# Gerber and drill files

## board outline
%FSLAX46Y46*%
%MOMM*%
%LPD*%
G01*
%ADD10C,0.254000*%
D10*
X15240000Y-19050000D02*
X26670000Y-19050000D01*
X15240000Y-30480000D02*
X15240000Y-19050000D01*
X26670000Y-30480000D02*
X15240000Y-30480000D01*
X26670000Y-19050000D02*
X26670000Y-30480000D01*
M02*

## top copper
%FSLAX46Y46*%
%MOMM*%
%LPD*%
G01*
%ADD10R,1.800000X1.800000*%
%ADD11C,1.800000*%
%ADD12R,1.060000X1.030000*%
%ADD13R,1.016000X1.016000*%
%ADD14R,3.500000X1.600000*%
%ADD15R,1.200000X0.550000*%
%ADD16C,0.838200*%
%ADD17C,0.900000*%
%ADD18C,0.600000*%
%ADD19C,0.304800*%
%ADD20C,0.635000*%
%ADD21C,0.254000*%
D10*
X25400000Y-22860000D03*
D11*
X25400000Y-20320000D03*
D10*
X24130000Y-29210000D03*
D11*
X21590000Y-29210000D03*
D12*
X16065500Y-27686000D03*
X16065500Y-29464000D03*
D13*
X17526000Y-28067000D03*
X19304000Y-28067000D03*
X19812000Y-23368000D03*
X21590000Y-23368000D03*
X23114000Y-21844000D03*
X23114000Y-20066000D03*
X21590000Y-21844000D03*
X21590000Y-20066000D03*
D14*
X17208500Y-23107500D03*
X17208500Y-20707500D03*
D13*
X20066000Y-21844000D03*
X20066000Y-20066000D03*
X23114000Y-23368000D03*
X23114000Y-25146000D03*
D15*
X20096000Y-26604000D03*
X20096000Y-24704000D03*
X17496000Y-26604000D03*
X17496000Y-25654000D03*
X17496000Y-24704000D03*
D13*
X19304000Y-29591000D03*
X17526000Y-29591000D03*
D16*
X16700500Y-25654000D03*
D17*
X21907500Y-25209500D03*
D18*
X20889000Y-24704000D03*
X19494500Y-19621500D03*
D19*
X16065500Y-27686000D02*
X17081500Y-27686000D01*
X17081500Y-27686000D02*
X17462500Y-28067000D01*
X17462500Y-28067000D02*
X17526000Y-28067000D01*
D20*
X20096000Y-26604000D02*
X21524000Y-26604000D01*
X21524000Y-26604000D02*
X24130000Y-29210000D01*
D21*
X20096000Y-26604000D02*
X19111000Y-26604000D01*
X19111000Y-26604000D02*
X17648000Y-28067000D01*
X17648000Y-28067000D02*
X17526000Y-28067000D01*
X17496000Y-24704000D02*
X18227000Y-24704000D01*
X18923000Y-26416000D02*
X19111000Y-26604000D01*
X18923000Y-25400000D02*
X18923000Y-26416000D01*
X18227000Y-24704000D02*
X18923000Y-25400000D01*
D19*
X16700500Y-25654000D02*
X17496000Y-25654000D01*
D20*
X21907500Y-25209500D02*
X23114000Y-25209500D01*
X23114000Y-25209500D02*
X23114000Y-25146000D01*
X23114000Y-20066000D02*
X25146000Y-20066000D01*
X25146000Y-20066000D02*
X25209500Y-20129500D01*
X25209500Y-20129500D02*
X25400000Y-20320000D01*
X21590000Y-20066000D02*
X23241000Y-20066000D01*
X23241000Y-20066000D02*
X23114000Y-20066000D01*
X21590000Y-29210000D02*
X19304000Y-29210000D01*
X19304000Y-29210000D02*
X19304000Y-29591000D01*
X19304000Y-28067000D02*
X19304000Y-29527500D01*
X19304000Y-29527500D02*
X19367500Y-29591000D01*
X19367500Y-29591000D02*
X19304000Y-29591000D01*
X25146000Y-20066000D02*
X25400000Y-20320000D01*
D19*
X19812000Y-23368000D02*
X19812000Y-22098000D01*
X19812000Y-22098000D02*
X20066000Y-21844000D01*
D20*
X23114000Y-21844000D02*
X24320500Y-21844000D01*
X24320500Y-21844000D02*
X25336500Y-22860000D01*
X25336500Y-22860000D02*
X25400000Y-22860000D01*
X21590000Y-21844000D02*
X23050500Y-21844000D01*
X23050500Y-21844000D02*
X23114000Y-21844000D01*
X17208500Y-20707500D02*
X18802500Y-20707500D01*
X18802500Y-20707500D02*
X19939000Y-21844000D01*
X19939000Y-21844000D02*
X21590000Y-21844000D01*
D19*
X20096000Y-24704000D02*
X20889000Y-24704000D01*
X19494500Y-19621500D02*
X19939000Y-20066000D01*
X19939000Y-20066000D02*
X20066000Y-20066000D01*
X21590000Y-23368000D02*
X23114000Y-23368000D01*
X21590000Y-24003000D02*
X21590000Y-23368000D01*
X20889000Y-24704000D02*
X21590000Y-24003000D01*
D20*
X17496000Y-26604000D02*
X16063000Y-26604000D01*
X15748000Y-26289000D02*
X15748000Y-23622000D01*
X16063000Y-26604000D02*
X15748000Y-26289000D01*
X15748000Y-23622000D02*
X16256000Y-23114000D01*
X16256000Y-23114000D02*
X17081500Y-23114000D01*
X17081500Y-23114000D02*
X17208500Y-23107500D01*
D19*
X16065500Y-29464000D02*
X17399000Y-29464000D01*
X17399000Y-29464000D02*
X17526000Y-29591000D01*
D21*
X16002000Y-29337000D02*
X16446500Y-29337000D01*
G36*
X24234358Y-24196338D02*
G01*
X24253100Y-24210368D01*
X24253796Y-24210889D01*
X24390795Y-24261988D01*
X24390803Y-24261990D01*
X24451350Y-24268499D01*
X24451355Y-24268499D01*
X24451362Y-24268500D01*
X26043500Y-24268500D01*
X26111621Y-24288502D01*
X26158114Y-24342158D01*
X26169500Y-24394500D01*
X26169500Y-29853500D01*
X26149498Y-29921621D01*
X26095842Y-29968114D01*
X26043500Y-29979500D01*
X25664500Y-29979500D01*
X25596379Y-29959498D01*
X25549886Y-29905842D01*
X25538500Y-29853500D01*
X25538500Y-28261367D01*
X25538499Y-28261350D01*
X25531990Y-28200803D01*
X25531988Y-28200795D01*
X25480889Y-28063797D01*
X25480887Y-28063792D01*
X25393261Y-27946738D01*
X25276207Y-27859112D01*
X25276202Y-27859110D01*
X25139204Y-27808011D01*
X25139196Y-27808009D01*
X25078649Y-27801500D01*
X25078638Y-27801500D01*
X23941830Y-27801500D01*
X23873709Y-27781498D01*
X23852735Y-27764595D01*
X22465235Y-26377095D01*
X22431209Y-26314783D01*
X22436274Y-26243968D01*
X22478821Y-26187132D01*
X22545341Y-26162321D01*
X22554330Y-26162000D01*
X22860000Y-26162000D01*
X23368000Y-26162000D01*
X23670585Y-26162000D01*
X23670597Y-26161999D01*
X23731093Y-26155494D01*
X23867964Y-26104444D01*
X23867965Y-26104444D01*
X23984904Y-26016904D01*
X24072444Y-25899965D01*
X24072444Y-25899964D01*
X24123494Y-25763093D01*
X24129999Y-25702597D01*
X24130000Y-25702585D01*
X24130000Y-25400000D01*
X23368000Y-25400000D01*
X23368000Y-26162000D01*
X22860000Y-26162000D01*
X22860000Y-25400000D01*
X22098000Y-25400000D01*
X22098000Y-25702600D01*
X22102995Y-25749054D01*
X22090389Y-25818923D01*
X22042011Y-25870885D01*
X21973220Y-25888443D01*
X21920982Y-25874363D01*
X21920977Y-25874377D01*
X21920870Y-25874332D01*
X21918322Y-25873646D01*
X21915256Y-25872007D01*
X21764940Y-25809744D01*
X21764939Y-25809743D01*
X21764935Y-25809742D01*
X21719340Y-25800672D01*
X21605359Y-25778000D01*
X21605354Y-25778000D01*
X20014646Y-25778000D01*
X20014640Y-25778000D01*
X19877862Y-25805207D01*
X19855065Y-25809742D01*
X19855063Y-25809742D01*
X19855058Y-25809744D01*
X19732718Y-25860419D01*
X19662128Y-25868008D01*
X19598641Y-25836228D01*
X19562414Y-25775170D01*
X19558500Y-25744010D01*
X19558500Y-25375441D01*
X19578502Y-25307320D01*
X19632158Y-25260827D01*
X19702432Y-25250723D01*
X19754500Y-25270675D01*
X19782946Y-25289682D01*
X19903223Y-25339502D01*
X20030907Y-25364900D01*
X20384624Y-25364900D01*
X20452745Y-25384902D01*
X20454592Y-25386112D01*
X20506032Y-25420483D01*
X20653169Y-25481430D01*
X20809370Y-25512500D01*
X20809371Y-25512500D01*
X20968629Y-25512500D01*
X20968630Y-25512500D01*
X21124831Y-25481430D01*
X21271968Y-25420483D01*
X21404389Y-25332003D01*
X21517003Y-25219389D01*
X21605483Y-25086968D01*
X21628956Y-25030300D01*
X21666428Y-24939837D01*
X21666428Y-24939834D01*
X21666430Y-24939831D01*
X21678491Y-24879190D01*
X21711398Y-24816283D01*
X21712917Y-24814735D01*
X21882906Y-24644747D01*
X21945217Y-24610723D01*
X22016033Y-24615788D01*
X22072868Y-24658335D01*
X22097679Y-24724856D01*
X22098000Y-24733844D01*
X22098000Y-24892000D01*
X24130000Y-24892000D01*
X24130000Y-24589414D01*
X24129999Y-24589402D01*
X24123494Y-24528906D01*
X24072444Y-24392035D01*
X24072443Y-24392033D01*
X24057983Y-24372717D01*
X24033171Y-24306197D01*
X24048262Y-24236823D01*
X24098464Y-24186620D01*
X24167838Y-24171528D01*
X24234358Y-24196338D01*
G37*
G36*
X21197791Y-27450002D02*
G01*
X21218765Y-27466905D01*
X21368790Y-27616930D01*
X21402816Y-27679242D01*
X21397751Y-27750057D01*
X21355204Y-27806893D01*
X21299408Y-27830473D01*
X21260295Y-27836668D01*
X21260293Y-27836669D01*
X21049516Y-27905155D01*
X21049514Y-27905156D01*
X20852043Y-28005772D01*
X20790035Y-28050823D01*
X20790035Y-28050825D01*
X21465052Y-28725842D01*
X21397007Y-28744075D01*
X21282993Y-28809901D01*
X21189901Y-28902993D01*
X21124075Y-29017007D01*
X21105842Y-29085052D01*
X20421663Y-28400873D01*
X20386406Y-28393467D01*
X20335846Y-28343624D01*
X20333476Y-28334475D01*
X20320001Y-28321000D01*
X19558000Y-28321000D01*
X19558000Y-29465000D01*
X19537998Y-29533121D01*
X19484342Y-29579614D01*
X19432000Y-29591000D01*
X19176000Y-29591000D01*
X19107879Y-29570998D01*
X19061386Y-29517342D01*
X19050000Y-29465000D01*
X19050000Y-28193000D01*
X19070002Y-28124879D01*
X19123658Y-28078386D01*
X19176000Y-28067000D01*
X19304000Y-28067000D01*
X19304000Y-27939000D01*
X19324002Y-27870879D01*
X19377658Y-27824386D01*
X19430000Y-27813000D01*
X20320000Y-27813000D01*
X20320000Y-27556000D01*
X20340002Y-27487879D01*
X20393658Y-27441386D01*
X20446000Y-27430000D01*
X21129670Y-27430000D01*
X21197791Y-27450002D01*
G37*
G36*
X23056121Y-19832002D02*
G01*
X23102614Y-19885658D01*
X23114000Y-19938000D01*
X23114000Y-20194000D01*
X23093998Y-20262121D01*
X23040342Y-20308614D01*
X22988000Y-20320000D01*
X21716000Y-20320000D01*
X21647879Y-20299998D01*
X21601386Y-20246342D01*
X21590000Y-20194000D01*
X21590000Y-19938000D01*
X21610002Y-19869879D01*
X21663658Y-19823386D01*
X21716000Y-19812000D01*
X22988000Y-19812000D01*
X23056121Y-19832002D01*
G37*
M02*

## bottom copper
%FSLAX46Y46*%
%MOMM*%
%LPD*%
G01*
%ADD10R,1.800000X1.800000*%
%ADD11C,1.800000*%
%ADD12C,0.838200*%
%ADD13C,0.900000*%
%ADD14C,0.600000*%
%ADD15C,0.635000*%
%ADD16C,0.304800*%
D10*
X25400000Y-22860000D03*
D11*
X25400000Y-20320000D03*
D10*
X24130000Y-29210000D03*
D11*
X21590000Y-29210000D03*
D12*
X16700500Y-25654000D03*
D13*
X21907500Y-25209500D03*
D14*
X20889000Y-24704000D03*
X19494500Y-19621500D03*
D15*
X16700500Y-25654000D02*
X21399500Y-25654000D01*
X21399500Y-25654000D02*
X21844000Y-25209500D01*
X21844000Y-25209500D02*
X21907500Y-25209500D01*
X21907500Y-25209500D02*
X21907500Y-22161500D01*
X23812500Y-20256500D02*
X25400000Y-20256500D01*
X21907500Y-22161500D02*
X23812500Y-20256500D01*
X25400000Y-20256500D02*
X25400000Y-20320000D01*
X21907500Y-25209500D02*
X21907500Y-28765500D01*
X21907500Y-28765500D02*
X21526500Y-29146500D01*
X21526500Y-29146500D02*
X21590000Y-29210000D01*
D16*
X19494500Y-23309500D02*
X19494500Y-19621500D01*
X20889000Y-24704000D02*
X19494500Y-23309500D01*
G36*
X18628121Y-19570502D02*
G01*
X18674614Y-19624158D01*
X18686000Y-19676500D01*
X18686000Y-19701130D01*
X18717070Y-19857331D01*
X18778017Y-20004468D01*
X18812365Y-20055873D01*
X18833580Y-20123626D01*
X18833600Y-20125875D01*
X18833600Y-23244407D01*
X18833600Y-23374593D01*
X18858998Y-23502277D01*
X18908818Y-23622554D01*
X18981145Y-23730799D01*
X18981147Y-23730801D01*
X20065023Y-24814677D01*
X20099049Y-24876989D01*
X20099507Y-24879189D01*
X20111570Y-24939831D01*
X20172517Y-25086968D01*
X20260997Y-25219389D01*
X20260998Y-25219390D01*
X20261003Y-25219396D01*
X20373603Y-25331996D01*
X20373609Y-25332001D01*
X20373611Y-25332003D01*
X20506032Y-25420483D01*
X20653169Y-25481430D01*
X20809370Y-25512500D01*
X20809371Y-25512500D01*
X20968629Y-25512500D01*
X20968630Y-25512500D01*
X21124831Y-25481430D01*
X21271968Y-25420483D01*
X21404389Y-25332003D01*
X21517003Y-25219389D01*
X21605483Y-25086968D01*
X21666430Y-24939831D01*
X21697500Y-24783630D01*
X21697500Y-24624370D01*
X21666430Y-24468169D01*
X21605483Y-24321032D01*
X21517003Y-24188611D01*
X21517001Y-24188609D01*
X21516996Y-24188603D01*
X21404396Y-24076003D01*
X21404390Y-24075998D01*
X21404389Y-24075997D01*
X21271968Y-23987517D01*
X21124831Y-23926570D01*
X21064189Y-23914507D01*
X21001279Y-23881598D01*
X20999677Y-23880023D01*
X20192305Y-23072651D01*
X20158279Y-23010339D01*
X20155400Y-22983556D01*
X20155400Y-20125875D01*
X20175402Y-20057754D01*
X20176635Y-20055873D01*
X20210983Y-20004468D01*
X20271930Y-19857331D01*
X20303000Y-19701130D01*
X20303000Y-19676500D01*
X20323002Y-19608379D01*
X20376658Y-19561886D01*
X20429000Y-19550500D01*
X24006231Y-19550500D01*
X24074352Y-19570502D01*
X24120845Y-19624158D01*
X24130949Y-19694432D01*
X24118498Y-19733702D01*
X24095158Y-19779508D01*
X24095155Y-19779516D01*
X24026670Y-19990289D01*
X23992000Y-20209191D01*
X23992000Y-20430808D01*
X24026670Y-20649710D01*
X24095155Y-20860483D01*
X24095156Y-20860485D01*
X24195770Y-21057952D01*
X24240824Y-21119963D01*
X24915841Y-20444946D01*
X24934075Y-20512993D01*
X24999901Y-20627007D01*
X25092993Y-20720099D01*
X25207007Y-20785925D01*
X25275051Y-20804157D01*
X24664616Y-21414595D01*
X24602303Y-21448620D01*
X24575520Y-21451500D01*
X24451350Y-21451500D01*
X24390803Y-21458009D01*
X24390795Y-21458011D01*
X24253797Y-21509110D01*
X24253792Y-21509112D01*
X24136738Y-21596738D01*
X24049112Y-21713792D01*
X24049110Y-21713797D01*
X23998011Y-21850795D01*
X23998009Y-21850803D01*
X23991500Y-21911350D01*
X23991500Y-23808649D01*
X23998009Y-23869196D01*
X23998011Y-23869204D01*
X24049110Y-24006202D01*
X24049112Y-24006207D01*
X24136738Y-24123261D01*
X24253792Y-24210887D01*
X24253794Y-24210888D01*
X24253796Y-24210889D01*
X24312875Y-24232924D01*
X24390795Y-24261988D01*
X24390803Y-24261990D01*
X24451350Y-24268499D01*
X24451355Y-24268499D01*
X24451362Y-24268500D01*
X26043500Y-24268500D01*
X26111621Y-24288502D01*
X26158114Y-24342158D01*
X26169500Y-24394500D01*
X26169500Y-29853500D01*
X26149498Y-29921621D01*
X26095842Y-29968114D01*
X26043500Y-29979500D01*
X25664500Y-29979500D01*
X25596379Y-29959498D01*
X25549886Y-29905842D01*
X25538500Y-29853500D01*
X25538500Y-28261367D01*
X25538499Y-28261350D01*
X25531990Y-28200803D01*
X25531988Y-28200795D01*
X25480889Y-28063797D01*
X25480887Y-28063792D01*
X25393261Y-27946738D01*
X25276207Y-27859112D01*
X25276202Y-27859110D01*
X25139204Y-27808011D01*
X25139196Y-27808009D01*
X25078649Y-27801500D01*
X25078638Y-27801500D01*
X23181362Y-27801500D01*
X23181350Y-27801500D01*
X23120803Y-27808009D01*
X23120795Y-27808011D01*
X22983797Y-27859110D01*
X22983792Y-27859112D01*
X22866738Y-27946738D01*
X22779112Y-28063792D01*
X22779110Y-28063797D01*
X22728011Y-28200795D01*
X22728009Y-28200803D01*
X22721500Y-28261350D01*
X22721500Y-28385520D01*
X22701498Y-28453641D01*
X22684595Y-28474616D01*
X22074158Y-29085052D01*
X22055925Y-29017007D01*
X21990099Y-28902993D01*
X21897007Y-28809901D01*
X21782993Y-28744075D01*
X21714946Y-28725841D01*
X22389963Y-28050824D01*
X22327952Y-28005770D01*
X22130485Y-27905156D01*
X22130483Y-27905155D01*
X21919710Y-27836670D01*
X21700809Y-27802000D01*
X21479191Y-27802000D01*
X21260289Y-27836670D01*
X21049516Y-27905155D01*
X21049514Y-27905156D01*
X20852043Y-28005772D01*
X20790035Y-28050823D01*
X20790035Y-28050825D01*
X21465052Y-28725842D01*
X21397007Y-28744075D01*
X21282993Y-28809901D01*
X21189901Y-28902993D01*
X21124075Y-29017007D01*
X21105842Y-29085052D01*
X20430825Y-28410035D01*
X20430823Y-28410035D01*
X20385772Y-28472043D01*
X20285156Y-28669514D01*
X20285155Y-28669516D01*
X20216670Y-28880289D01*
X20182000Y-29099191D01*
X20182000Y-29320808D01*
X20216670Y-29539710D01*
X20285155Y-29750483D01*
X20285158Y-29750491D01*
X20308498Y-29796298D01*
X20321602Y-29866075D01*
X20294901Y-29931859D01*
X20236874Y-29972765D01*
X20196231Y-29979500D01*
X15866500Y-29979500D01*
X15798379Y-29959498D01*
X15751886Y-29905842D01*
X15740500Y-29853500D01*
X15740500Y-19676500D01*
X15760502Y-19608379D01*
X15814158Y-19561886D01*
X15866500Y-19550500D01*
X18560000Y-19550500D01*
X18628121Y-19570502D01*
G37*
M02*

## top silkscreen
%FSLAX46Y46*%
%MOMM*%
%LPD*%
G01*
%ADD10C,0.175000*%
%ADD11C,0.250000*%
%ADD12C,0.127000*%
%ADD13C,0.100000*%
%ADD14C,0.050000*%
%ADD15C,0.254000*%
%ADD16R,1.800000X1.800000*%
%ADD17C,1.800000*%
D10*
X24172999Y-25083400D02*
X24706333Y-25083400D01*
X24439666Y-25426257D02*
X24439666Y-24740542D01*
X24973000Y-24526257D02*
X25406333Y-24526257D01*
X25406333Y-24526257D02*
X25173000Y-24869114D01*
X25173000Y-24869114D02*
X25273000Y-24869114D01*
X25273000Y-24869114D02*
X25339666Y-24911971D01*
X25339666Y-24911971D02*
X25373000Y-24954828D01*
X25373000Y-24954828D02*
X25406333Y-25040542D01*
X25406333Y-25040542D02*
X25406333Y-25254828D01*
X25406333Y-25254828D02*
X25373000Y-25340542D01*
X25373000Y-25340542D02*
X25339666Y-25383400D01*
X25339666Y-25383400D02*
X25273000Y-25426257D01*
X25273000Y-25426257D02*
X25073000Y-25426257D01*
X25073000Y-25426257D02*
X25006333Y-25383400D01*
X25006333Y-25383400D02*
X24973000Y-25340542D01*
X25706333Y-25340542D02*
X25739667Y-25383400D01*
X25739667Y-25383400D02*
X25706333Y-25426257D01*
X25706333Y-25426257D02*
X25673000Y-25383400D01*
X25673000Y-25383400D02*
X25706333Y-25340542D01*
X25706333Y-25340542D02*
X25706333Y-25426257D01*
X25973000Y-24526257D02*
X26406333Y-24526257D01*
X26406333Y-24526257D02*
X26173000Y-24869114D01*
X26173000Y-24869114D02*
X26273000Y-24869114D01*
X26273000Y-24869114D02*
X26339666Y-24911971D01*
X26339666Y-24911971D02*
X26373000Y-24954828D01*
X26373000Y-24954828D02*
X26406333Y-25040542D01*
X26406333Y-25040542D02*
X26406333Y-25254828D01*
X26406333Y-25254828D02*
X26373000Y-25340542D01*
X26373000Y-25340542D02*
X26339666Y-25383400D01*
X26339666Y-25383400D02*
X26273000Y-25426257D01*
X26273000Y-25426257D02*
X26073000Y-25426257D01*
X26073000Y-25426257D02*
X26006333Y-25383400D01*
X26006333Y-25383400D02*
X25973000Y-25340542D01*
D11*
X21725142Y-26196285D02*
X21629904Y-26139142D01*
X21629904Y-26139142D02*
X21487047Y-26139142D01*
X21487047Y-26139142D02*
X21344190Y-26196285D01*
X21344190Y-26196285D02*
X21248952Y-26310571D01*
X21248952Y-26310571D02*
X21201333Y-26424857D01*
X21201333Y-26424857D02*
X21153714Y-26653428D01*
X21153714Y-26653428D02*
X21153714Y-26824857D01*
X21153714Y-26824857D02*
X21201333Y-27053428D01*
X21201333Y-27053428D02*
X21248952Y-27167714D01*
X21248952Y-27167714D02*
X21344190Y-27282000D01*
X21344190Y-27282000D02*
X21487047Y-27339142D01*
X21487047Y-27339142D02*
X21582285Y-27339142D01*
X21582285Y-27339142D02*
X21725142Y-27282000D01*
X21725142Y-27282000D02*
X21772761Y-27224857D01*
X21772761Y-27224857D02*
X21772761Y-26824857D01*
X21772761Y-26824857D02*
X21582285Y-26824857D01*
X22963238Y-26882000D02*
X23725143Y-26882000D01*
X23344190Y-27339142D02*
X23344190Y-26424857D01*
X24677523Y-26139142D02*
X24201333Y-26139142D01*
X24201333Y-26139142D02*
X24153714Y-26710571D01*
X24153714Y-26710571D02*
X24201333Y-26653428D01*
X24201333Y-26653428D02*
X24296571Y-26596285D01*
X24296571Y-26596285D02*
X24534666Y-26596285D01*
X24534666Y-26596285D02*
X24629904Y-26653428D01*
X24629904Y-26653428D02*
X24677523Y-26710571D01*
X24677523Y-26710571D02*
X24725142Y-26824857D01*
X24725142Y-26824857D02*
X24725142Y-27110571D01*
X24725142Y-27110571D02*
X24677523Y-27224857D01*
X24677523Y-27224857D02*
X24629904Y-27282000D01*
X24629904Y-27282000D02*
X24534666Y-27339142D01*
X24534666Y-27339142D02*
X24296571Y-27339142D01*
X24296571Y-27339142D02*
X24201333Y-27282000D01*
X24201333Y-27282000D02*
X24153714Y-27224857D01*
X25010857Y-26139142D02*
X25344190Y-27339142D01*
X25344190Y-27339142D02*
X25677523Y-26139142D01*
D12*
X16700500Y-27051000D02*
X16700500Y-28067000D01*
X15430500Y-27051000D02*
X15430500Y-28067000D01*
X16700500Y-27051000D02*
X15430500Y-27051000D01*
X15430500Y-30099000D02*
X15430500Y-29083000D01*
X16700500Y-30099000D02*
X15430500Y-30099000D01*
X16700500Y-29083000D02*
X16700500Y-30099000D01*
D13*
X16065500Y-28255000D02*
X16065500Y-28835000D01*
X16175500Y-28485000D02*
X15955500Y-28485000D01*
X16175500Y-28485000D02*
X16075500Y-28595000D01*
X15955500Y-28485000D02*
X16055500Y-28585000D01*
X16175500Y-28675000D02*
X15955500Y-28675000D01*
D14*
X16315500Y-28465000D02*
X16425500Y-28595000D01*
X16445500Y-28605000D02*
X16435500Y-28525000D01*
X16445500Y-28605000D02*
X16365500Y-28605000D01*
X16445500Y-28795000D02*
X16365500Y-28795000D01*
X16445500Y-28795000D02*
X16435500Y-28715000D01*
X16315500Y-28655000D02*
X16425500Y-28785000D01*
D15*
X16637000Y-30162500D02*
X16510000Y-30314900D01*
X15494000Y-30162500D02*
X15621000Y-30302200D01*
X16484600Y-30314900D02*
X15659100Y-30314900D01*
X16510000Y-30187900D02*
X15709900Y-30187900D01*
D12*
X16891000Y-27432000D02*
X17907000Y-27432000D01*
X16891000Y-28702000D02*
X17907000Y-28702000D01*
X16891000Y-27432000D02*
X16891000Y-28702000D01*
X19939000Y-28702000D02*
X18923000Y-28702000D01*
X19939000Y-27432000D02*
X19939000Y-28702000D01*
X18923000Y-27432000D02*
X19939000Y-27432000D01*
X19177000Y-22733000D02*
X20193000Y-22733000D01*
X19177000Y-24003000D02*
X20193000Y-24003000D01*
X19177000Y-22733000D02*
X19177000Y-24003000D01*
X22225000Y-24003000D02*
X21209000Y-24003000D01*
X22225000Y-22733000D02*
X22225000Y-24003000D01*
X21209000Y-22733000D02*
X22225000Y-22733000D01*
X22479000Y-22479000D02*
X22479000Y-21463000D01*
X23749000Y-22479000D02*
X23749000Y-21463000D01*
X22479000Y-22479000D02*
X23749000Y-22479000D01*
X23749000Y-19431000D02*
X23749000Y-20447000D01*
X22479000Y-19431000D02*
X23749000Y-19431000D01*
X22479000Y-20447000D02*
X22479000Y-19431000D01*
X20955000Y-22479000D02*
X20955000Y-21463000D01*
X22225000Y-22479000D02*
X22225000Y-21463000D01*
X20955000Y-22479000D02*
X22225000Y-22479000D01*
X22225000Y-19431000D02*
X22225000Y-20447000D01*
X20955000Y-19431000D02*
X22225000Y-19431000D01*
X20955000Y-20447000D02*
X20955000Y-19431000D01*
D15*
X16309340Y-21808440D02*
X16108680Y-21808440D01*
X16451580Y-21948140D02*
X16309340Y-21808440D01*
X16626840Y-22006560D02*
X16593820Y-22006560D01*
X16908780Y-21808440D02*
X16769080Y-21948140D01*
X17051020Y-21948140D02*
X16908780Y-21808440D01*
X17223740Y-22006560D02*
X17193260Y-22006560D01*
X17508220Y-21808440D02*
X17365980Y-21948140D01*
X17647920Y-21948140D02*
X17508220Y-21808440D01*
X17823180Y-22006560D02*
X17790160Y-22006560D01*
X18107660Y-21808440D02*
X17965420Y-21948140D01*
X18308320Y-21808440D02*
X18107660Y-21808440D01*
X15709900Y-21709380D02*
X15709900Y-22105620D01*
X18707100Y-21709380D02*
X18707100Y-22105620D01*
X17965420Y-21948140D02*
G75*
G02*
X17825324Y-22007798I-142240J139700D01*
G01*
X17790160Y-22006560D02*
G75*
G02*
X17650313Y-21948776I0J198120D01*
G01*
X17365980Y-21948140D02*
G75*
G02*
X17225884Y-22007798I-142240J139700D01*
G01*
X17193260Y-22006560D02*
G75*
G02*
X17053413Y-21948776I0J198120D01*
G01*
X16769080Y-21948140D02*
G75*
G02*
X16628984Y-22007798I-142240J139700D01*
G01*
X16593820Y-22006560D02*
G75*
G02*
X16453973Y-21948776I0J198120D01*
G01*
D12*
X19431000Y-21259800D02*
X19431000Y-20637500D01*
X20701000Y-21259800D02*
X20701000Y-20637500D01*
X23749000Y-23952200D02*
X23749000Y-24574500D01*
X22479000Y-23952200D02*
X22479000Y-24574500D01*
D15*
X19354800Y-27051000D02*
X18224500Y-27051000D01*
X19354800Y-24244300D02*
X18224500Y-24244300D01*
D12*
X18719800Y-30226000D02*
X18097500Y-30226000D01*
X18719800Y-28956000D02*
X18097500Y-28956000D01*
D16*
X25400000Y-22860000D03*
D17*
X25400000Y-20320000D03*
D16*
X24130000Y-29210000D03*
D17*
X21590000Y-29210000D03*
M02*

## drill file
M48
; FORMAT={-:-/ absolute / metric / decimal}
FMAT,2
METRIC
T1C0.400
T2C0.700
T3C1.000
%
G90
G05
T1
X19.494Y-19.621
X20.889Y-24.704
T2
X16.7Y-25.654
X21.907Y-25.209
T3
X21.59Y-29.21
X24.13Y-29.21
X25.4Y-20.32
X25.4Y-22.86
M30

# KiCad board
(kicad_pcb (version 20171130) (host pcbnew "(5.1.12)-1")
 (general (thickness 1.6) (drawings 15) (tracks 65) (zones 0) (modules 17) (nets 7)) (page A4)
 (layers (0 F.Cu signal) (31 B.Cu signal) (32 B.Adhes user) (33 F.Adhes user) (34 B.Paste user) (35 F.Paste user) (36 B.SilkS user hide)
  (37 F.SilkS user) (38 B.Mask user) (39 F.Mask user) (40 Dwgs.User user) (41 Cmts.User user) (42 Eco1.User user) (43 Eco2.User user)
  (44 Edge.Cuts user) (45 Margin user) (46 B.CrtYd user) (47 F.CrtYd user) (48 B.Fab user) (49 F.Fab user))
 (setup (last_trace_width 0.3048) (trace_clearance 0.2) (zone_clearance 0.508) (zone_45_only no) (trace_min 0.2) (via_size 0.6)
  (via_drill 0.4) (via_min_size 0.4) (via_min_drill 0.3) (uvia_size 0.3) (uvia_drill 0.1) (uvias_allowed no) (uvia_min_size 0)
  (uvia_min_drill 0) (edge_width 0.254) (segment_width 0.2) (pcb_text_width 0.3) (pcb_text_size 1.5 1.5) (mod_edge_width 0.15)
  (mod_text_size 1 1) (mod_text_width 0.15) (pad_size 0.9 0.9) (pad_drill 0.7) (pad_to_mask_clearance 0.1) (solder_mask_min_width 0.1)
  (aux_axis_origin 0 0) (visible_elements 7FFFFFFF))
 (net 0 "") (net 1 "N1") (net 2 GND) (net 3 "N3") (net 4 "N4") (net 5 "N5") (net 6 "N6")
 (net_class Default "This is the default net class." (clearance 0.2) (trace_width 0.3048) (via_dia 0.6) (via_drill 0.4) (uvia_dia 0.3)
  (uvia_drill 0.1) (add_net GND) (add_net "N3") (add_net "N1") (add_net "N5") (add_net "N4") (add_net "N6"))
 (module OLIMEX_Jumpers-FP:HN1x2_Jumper (layer F.Cu) (at 25.4 21.59 90)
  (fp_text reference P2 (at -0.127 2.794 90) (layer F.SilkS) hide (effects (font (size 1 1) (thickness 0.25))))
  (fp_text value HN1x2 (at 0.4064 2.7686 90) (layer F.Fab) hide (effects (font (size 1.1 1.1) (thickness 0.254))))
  (pad 1 thru_hole rect (at -1.27 0 180) (size 1.8 1.8) (drill 1) (layers *.Cu *.Mask F.SilkS) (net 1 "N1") (solder_mask_margin 0.0508)
   (solder_paste_margin -0.0508))
  (pad 2 thru_hole circle (at 1.27 0 180) (size 1.8 1.8) (drill 1) (layers *.Cu *.Mask F.SilkS) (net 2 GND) (solder_mask_margin 0.0508)
   (solder_paste_margin -0.0508)))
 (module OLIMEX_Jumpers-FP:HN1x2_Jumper (layer F.Cu) (at 22.86 29.21 180)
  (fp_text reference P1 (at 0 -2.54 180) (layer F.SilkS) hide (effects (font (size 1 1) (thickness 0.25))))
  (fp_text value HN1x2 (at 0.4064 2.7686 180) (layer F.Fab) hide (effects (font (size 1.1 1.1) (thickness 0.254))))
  (pad 1 thru_hole rect (at -1.27 0 270) (size 1.8 1.8) (drill 1) (layers *.Cu *.Mask F.SilkS) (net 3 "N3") (solder_mask_margin 0.0508)
   (solder_paste_margin -0.0508))
  (pad 2 thru_hole circle (at 1.27 0 270) (size 1.8 1.8) (drill 1) (layers *.Cu *.Mask F.SilkS) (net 2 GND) (solder_mask_margin 0.0508)
   (solder_paste_margin -0.0508)))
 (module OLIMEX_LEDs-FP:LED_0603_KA (layer F.Cu) (at 16.0655 28.575 270)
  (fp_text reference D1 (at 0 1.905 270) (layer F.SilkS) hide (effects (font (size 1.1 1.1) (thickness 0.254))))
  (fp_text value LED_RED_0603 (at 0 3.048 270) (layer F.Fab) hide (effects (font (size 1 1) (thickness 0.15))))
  (fp_line (start -1.524 -0.635) (end -0.508 -0.635) (layer F.SilkS) (width 0.127))
  (fp_line (start -1.524 0.635) (end -0.508 0.635) (layer F.SilkS) (width 0.127))
  (fp_line (start -1.524 -0.635) (end -1.524 0.635) (layer F.SilkS) (width 0.127))
  (fp_line (start 1.524 0.635) (end 0.508 0.635) (layer F.SilkS) (width 0.127))
  (fp_line (start 1.524 -0.635) (end 1.524 0.635) (layer F.SilkS) (width 0.127))
  (fp_line (start 0.508 -0.635) (end 1.524 -0.635) (layer F.SilkS) (width 0.127))
  (fp_line (start -0.32 0) (end 0.26 0) (layer F.SilkS) (width 0.1))
  (fp_line (start -0.09 -0.11) (end -0.09 0.11) (layer F.SilkS) (width 0.1))
  (fp_line (start -0.09 -0.11) (end 0.02 -0.01) (layer F.SilkS) (width 0.1))
  (fp_line (start -0.09 0.11) (end 0.01 0.01) (layer F.SilkS) (width 0.1))
  (fp_line (start 0.1 -0.11) (end 0.1 0.11) (layer F.SilkS) (width 0.1))
  (fp_line (start -0.11 -0.25) (end 0.02 -0.36) (layer F.SilkS) (width 0.05))
  (fp_line (start 0.03 -0.38) (end -0.05 -0.37) (layer F.SilkS) (width 0.05))
  (fp_line (start 0.03 -0.38) (end 0.03 -0.3) (layer F.SilkS) (width 0.05))
  (fp_line (start 0.22 -0.38) (end 0.22 -0.3) (layer F.SilkS) (width 0.05))
  (fp_line (start 0.22 -0.38) (end 0.14 -0.37) (layer F.SilkS) (width 0.05))
  (fp_line (start 0.08 -0.25) (end 0.21 -0.36) (layer F.SilkS) (width 0.05))
  (fp_line (start 1.5875 -0.5715) (end 1.7399 -0.4445) (layer F.SilkS) (width 0.254))
  (fp_line (start 1.5875 0.5715) (end 1.7272 0.4445) (layer F.SilkS) (width 0.254))
  (fp_line (start 1.7399 -0.4191) (end 1.7399 0.4064) (layer F.SilkS) (width 0.254))
  (fp_line (start 1.6129 -0.4445) (end 1.6129 0.3556) (layer F.SilkS) (width 0.254))
  (pad 2 smd rect (at -0.889 0 270) (size 1.03 1.06) (layers F.Cu F.Paste F.Mask) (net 3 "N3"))
  (pad 1 smd rect (at 0.889 0 270) (size 1.03 1.06) (layers F.Cu F.Paste F.Mask) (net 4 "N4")))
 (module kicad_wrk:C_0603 (layer F.Cu) (at 18.415 28.067)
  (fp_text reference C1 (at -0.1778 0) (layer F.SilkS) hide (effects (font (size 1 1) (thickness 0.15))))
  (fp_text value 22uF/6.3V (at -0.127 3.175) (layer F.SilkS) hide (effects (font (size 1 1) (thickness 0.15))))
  (fp_line (start -1.524 -0.635) (end -0.508 -0.635) (layer F.SilkS) (width 0.127))
  (fp_line (start -1.524 0.635) (end -0.508 0.635) (layer F.SilkS) (width 0.127))
  (fp_line (start -1.524 -0.635) (end -1.524 0.635) (layer F.SilkS) (width 0.127))
  (fp_line (start 1.524 0.635) (end 0.508 0.635) (layer F.SilkS) (width 0.127))
  (fp_line (start 1.524 -0.635) (end 1.524 0.635) (layer F.SilkS) (width 0.127))
  (fp_line (start 0.508 -0.635) (end 1.524 -0.635) (layer F.SilkS) (width 0.127))
  (pad 1 smd rect (at -0.889 0) (size 1.016 1.016) (layers F.Cu F.Paste F.Mask) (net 3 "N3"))
  (pad 2 smd rect (at 0.889 0) (size 1.016 1.016) (layers F.Cu F.Paste F.Mask) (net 2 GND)))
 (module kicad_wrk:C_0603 (layer F.Cu) (at 20.701 23.368)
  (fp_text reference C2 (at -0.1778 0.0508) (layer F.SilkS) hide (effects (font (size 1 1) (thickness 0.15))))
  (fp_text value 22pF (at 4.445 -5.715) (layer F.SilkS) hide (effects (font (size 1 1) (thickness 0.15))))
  (fp_line (start -1.524 -0.635) (end -0.508 -0.635) (layer F.SilkS) (width 0.127))
  (fp_line (start -1.524 0.635) (end -0.508 0.635) (layer F.SilkS) (width 0.127))
  (fp_line (start -1.524 -0.635) (end -1.524 0.635) (layer F.SilkS) (width 0.127))
  (fp_line (start 1.524 0.635) (end 0.508 0.635) (layer F.SilkS) (width 0.127))
  (fp_line (start 1.524 -0.635) (end 1.524 0.635) (layer F.SilkS) (width 0.127))
  (fp_line (start 0.508 -0.635) (end 1.524 -0.635) (layer F.SilkS) (width 0.127))
  (pad 1 smd rect (at -0.889 0) (size 1.016 1.016) (layers F.Cu F.Paste F.Mask) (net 1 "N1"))
  (pad 2 smd rect (at 0.889 0) (size 1.016 1.016) (layers F.Cu F.Paste F.Mask) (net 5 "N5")))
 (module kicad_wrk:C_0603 (layer F.Cu) (at 23.114 20.955 90)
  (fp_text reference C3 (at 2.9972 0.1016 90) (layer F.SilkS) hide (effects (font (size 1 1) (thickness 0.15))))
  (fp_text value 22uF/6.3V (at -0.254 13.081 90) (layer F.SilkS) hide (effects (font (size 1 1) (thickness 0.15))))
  (fp_line (start -1.524 -0.635) (end -0.508 -0.635) (layer F.SilkS) (width 0.127))
  (fp_line (start -1.524 0.635) (end -0.508 0.635) (layer F.SilkS) (width 0.127))
  (fp_line (start -1.524 -0.635) (end -1.524 0.635) (layer F.SilkS) (width 0.127))
  (fp_line (start 1.524 0.635) (end 0.508 0.635) (layer F.SilkS) (width 0.127))
  (fp_line (start 1.524 -0.635) (end 1.524 0.635) (layer F.SilkS) (width 0.127))
  (fp_line (start 0.508 -0.635) (end 1.524 -0.635) (layer F.SilkS) (width 0.127))
  (pad 1 smd rect (at -0.889 0 90) (size 1.016 1.016) (layers F.Cu F.Paste F.Mask) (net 1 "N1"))
  (pad 2 smd rect (at 0.889 0 90) (size 1.016 1.016) (layers F.Cu F.Paste F.Mask) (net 2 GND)))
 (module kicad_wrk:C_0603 (layer F.Cu) (at 21.59 20.955 90)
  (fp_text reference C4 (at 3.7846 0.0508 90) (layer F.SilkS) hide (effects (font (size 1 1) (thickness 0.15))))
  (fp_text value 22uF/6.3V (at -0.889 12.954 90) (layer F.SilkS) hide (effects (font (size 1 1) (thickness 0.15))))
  (fp_line (start -1.524 -0.635) (end -0.508 -0.635) (layer F.SilkS) (width 0.127))
  (fp_line (start -1.524 0.635) (end -0.508 0.635) (layer F.SilkS) (width 0.127))
  (fp_line (start -1.524 -0.635) (end -1.524 0.635) (layer F.SilkS) (width 0.127))
  (fp_line (start 1.524 0.635) (end 0.508 0.635) (layer F.SilkS) (width 0.127))
  (fp_line (start 1.524 -0.635) (end 1.524 0.635) (layer F.SilkS) (width 0.127))
  (fp_line (start 0.508 -0.635) (end 1.524 -0.635) (layer F.SilkS) (width 0.127))
  (pad 1 smd rect (at -0.889 0 90) (size 1.016 1.016) (layers F.Cu F.Paste F.Mask) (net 1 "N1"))
  (pad 2 smd rect (at 0.889 0 90) (size 1.016 1.016) (layers F.Cu F.Paste F.Mask) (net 2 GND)))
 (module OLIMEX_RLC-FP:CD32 (layer F.Cu) (at 17.2085 21.9075 90)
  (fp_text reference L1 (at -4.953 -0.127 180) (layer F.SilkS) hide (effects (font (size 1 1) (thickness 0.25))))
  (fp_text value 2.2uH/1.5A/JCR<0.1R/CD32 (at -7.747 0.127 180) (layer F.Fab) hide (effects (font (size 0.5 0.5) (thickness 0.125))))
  (fp_line (start 0.09906 -0.89916) (end 0.09906 -1.09982) (layer F.SilkS) (width 0.254))
  (fp_line (start -0.04064 -0.75692) (end 0.09906 -0.89916) (layer F.SilkS) (width 0.254))
  (fp_line (start -0.09906 -0.58166) (end -0.09906 -0.61468) (layer F.SilkS) (width 0.254))
  (fp_line (start 0.09906 -0.29972) (end -0.04064 -0.43942) (layer F.SilkS) (width 0.254))
  (fp_line (start -0.04064 -0.15748) (end 0.09906 -0.29972) (layer F.SilkS) (width 0.254))
  (fp_line (start -0.09906 0.01524) (end -0.09906 -0.01524) (layer F.SilkS) (width 0.254))
  (fp_line (start 0.09906 0.29972) (end -0.04064 0.15748) (layer F.SilkS) (width 0.254))
  (fp_line (start -0.04064 0.43942) (end 0.09906 0.29972) (layer F.SilkS) (width 0.254))
  (fp_line (start -0.09906 0.61468) (end -0.09906 0.58166) (layer F.SilkS) (width 0.254))
  (fp_line (start 0.09906 0.89916) (end -0.04064 0.75692) (layer F.SilkS) (width 0.254))
  (fp_line (start 0.09906 1.09982) (end 0.09906 0.89916) (layer F.SilkS) (width 0.254))
  (fp_line (start 0.19812 -1.4986) (end -0.19812 -1.4986) (layer F.SilkS) (width 0.254))
  (fp_line (start 0.19812 1.4986) (end -0.19812 1.4986) (layer F.SilkS) (width 0.254))
  (fp_arc (start 0.09906 0.61468) (end -0.04064 0.75692) (angle 44.9) (layer F.SilkS) (width 0.254))
  (fp_arc (start 0.09906 0.58166) (end -0.09906 0.58166) (angle 44.9) (layer F.SilkS) (width 0.254))
  (fp_arc (start 0.09906 0.01524) (end -0.04064 0.15748) (angle 44.9) (layer F.SilkS) (width 0.254))
  (fp_arc (start 0.09906 -0.01524) (end -0.09906 -0.01524) (angle 44.9) (layer F.SilkS) (width 0.254))
  (fp_arc (start 0.09906 -0.58166) (end -0.04064 -0.43942) (angle 44.9) (layer F.SilkS) (width 0.254))
  (fp_arc (start 0.09906 -0.61468) (end -0.09906 -0.61468) (angle 44.9) (layer F.SilkS) (width 0.254))
  (pad 1 smd rect (at -1.2 0 180) (size 3.5 1.6) (layers F.Cu F.Paste F.Mask) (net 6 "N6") (solder_mask_margin 0.0508)
   (solder_paste_margin -0.0508) (clearance 0.0508))
  (pad 2 smd rect (at 1.2 0 180) (size 3.5 1.6) (layers F.Cu F.Paste F.Mask) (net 1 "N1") (solder_mask_margin 0.0508)
   (solder_paste_margin -0.0508) (clearance 0.0508)))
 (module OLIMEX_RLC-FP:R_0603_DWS (layer F.Cu) (at 20.066 20.955 90)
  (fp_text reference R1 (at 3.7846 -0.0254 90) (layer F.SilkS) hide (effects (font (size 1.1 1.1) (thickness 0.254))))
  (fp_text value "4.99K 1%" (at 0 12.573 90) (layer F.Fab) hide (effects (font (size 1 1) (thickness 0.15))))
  (fp_line (start -0.3048 -0.635) (end 0.3175 -0.635) (layer F.SilkS) (width 0.127))
  (fp_line (start -0.3048 0.635) (end 0.3175 0.635) (layer F.SilkS) (width 0.127))
  (pad 1 smd rect (at -0.889 0 90) (size 1.016 1.016) (layers F.Cu F.Paste F.Mask) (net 1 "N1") (solder_mask_margin 0.0508)
   (solder_paste_margin -0.0508) (clearance 0.0508))
  (pad 2 smd rect (at 0.889 0 90) (size 1.016 1.016) (layers F.Cu F.Paste F.Mask) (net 5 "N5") (solder_mask_margin 0.0508)
   (solder_paste_margin -0.0508) (clearance 0.0508)))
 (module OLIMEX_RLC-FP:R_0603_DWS (layer F.Cu) (at 23.114 24.257 270)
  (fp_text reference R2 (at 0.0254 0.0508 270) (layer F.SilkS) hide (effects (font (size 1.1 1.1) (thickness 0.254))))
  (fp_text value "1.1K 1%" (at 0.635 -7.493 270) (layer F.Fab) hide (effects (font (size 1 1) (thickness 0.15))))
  (fp_line (start -0.3048 -0.635) (end 0.3175 -0.635) (layer F.SilkS) (width 0.127))
  (fp_line (start -0.3048 0.635) (end 0.3175 0.635) (layer F.SilkS) (width 0.127))
  (pad 1 smd rect (at -0.889 0 270) (size 1.016 1.016) (layers F.Cu F.Paste F.Mask) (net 5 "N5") (solder_mask_margin 0.0508)
   (solder_paste_margin -0.0508) (clearance 0.0508))
  (pad 2 smd rect (at 0.889 0 270) (size 1.016 1.016) (layers F.Cu F.Paste F.Mask) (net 2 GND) (solder_mask_margin 0.0508)
   (solder_paste_margin -0.0508) (clearance 0.0508)))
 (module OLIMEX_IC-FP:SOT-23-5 (layer F.Cu) (at 18.796 25.654 180)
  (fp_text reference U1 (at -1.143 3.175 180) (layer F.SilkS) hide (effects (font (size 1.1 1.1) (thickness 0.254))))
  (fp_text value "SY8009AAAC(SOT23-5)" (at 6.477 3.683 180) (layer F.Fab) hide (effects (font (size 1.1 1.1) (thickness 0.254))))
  (fp_line (start -0.5588 -1.397) (end 0.5715 -1.397) (layer F.SilkS) (width 0.254))
  (fp_line (start -0.5588 1.4097) (end 0.5715 1.4097) (layer F.SilkS) (width 0.254))
  (pad 4 smd rect (at -1.3 -0.95 180) (size 1.2 0.55) (layers F.Cu F.Paste F.Mask) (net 3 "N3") (solder_mask_margin 0.0508)
   (solder_paste_margin -0.0508) (clearance 0.0508))
  (pad 5 smd rect (at -1.3 0.95 180) (size 1.2 0.55) (layers F.Cu F.Paste F.Mask) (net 5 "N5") (solder_mask_margin 0.0508)
   (solder_paste_margin -0.0508) (clearance 0.0508))
  (pad 3 smd rect (at 1.3 -0.95 180) (size 1.2 0.55) (layers F.Cu F.Paste F.Mask) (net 6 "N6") (solder_mask_margin 0.0508)
   (solder_paste_margin -0.0508) (clearance 0.0508))
  (pad 2 smd rect (at 1.3 0 180) (size 1.2 0.55) (layers F.Cu F.Paste F.Mask) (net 2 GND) (solder_mask_margin 0.0508)
   (solder_paste_margin -0.0508) (clearance 0.0508))
  (pad 1 smd rect (at 1.3 0.95 180) (size 1.2 0.55) (layers F.Cu F.Paste F.Mask) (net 3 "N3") (solder_mask_margin 0.0508)
   (solder_paste_margin -0.0508) (clearance 0.0508)))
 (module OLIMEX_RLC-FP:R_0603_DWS (layer F.Cu) (at 18.415 29.591 180)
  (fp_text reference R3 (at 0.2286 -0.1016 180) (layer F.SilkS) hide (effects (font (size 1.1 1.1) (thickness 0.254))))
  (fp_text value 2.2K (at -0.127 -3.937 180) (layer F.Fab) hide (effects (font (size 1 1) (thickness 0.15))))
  (fp_line (start -0.3048 -0.635) (end 0.3175 -0.635) (layer F.SilkS) (width 0.127))
  (fp_line (start -0.3048 0.635) (end 0.3175 0.635) (layer F.SilkS) (width 0.127))
  (pad 1 smd rect (at -0.889 0 180) (size 1.016 1.016) (layers F.Cu F.Paste F.Mask) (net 2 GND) (solder_mask_margin 0.0508)
   (solder_paste_margin -0.0508) (clearance 0.0508))
  (pad 2 smd rect (at 0.889 0 180) (size 1.016 1.016) (layers F.Cu F.Paste F.Mask) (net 4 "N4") (solder_mask_margin 0.0508)
   (solder_paste_margin -0.0508) (clearance 0.0508)))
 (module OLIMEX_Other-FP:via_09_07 (layer F.Cu) (at 16.7005 25.654)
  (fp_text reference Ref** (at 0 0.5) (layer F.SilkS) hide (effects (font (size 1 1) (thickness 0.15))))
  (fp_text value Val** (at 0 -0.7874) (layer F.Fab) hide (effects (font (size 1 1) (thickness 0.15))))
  (pad 0 thru_hole circle (at 0 0) (size 0.8382 0.8382) (drill 0.7) (layers *.Cu) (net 2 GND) (zone_connect 2)))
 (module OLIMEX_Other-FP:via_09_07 (layer F.Cu) (at 21.9075 25.273)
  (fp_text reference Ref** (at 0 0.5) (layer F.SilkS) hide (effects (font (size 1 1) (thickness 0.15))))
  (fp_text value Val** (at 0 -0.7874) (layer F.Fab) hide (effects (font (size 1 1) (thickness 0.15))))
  (pad 0 thru_hole circle (at 0 -0.0635) (size 0.9 0.9) (drill 0.7) (layers *.Cu) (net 2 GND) (zone_connect 2)))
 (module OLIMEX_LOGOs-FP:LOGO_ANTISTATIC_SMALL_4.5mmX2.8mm (layer B.Cu) (at 18.4785 28.194 180)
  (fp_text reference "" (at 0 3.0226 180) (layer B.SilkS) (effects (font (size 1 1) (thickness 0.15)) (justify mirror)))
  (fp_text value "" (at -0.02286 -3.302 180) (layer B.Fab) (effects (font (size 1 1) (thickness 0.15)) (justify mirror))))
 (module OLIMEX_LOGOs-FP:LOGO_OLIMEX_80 (layer B.Cu) (at 19.939 24.3205 180)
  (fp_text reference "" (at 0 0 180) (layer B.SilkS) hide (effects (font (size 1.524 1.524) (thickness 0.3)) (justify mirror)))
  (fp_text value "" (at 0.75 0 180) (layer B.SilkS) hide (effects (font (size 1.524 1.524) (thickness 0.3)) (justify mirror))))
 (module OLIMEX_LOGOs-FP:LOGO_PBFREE (layer B.Cu) (at 18.669 21.3995 180)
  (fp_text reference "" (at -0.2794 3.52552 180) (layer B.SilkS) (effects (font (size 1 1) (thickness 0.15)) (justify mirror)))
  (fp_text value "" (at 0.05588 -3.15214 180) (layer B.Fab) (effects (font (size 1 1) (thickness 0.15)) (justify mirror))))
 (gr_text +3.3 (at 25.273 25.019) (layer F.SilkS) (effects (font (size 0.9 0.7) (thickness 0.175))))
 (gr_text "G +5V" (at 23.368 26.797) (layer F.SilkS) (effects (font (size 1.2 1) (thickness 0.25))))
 (gr_line (start 15.24 19.05) (end 26.67 19.05) (angle 90) (layer Edge.Cuts) (width 0.254))
 (gr_line (start 15.24 30.48) (end 15.24 19.05) (angle 90) (layer Edge.Cuts) (width 0.254))
 (gr_line (start 26.67 30.48) (end 15.24 30.48) (angle 90) (layer Edge.Cuts) (width 0.254))
 (gr_line (start 26.67 19.05) (end 26.67 30.48) (angle 90) (layer Edge.Cuts) (width 0.254))
 (segment (start 16.0655 27.686) (end 17.0815 27.686) (width 0.3048) (layer F.Cu) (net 3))
 (segment (start 17.0815 27.686) (end 17.4625 28.067) (width 0.3048) (layer F.Cu) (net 3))
 (segment (start 17.4625 28.067) (end 17.526 28.067) (width 0.3048) (layer F.Cu) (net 3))
 (segment (start 20.096 26.604) (end 21.524 26.604) (width 0.635) (layer F.Cu) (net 3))
 (segment (start 21.524 26.604) (end 24.13 29.21) (width 0.635) (layer F.Cu) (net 3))
 (segment (start 20.096 26.604) (end 19.111 26.604) (width 0.254) (layer F.Cu) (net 3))
 (segment (start 19.111 26.604) (end 17.648 28.067) (width 0.254) (layer F.Cu) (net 3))
 (segment (start 17.648 28.067) (end 17.526 28.067) (width 0.254) (layer F.Cu) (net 3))
 (segment (start 17.496 24.704) (end 18.227 24.704) (width 0.254) (layer F.Cu) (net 3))
 (segment (start 18.923 26.416) (end 19.111 26.604) (width 0.254) (layer F.Cu) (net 3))
 (segment (start 18.923 25.4) (end 18.923 26.416) (width 0.254) (layer F.Cu) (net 3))
 (segment (start 18.227 24.704) (end 18.923 25.4) (width 0.254) (layer F.Cu) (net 3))
 (segment (start 16.7005 25.654) (end 17.496 25.654) (width 0.3048) (layer F.Cu) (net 2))
 (segment (start 16.7005 25.654) (end 21.3995 25.654) (width 0.635) (layer B.Cu) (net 2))
 (segment (start 21.3995 25.654) (end 21.844 25.2095) (width 0.635) (layer B.Cu) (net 2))
 (segment (start 21.844 25.2095) (end 21.9075 25.2095) (width 0.635) (layer B.Cu) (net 2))
 (segment (start 21.9075 25.2095) (end 21.9075 22.1615) (width 0.635) (layer B.Cu) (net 2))
 (segment (start 23.8125 20.2565) (end 25.4 20.2565) (width 0.635) (layer B.Cu) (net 2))
 (segment (start 21.9075 22.1615) (end 23.8125 20.2565) (width 0.635) (layer B.Cu) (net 2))
 (segment (start 25.4 20.2565) (end 25.4 20.32) (width 0.635) (layer B.Cu) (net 2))
 (segment (start 21.9075 25.2095) (end 21.9075 28.7655) (width 0.635) (layer B.Cu) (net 2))
 (segment (start 21.9075 28.7655) (end 21.5265 29.1465) (width 0.635) (layer B.Cu) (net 2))
 (segment (start 21.5265 29.1465) (end 21.59 29.21) (width 0.635) (layer B.Cu) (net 2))
 (segment (start 21.9075 25.2095) (end 23.114 25.2095) (width 0.635) (layer F.Cu) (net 2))
 (segment (start 23.114 25.2095) (end 23.114 25.146) (width 0.635) (layer F.Cu) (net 2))
 (segment (start 23.114 20.066) (end 25.146 20.066) (width 0.635) (layer F.Cu) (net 2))
 (segment (start 25.146 20.066) (end 25.2095 20.1295) (width 0.635) (layer F.Cu) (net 2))
 (segment (start 25.2095 20.1295) (end 25.4 20.32) (width 0.635) (layer F.Cu) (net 2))
 (segment (start 21.59 20.066) (end 23.241 20.066) (width 0.635) (layer F.Cu) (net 2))
 (segment (start 23.241 20.066) (end 23.114 20.066) (width 0.635) (layer F.Cu) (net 2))
 (segment (start 21.59 29.21) (end 19.304 29.21) (width 0.635) (layer F.Cu) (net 2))
 (segment (start 19.304 29.21) (end 19.304 29.591) (width 0.635) (layer F.Cu) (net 2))
 (segment (start 19.304 28.067) (end 19.304 29.5275) (width 0.635) (layer F.Cu) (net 2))
 (segment (start 19.304 29.5275) (end 19.3675 29.591) (width 0.635) (layer F.Cu) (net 2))
 (segment (start 19.3675 29.591) (end 19.304 29.591) (width 0.635) (layer F.Cu) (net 2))
 (segment (start 25.146 20.066) (end 25.4 20.32) (width 0.635) (layer F.Cu) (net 2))
 (segment (start 19.812 23.368) (end 19.812 22.098) (width 0.3048) (layer F.Cu) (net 1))
 (segment (start 19.812 22.098) (end 20.066 21.844) (width 0.3048) (layer F.Cu) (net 1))
 (segment (start 23.114 21.844) (end 24.3205 21.844) (width 0.635) (layer F.Cu) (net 1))
 (segment (start 24.3205 21.844) (end 25.3365 22.86) (width 0.635) (layer F.Cu) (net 1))
 (segment (start 25.3365 22.86) (end 25.4 22.86) (width 0.635) (layer F.Cu) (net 1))
 (segment (start 21.59 21.844) (end 23.0505 21.844) (width 0.635) (layer F.Cu) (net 1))
 (segment (start 23.0505 21.844) (end 23.114 21.844) (width 0.635) (layer F.Cu) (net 1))
 (segment (start 17.2085 20.7075) (end 18.8025 20.7075) (width 0.635) (layer F.Cu) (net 1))
 (segment (start 18.8025 20.7075) (end 19.939 21.844) (width 0.635) (layer F.Cu) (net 1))
 (segment (start 19.939 21.844) (end 21.59 21.844) (width 0.635) (layer F.Cu) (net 1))
 (segment (start 20.096 24.704) (end 20.889 24.704) (width 0.3048) (layer F.Cu) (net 5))
 (via (at 20.889 24.704) (size 0.6) (layers F.Cu B.Cu) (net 5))
 (segment (start 19.4945 19.6215) (end 19.939 20.066) (width 0.3048) (layer F.Cu) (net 5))
 (via (at 19.4945 19.6215) (size 0.6) (layers F.Cu B.Cu) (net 5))
 (segment (start 19.4945 23.3095) (end 19.4945 19.6215) (width 0.3048) (layer B.Cu) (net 5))
 (segment (start 20.889 24.704) (end 19.4945 23.3095) (width 0.3048) (layer B.Cu) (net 5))
 (segment (start 19.939 20.066) (end 20.066 20.066) (width 0.3048) (layer F.Cu) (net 5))
 (segment (start 21.59 23.368) (end 23.114 23.368) (width 0.3048) (layer F.Cu) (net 5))
 (segment (start 21.59 24.003) (end 21.59 23.368) (width 0.3048) (layer F.Cu) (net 5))
 (segment (start 20.889 24.704) (end 21.59 24.003) (width 0.3048) (layer F.Cu) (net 5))
 (segment (start 17.496 26.604) (end 16.063 26.604) (width 0.635) (layer F.Cu) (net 6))
 (segment (start 15.748 26.289) (end 15.748 23.622) (width 0.635) (layer F.Cu) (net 6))
 (segment (start 16.063 26.604) (end 15.748 26.289) (width 0.635) (layer F.Cu) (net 6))
 (segment (start 15.748 23.622) (end 16.256 23.114) (width 0.635) (layer F.Cu) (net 6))
 (segment (start 16.256 23.114) (end 17.0815 23.114) (width 0.635) (layer F.Cu) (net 6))
 (segment (start 17.0815 23.114) (end 17.2085 23.1075) (width 0.635) (layer F.Cu) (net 6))
 (segment (start 16.0655 29.464) (end 17.399 29.464) (width 0.3048) (layer F.Cu) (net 4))
 (segment (start 17.399 29.464) (end 17.526 29.591) (width 0.3048) (layer F.Cu) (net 4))
 (segment (start 16.002 29.337) (end 16.4465 29.337) (width 0.254) (layer F.Cu) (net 4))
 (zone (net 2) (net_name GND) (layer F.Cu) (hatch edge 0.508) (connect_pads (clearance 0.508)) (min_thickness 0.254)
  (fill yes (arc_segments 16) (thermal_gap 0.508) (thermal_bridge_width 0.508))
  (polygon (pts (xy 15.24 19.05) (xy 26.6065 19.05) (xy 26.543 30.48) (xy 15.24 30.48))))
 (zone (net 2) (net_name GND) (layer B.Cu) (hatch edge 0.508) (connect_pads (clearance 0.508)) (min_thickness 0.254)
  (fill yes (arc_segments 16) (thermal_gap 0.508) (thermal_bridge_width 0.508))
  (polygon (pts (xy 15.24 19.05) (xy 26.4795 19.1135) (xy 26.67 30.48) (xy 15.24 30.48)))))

